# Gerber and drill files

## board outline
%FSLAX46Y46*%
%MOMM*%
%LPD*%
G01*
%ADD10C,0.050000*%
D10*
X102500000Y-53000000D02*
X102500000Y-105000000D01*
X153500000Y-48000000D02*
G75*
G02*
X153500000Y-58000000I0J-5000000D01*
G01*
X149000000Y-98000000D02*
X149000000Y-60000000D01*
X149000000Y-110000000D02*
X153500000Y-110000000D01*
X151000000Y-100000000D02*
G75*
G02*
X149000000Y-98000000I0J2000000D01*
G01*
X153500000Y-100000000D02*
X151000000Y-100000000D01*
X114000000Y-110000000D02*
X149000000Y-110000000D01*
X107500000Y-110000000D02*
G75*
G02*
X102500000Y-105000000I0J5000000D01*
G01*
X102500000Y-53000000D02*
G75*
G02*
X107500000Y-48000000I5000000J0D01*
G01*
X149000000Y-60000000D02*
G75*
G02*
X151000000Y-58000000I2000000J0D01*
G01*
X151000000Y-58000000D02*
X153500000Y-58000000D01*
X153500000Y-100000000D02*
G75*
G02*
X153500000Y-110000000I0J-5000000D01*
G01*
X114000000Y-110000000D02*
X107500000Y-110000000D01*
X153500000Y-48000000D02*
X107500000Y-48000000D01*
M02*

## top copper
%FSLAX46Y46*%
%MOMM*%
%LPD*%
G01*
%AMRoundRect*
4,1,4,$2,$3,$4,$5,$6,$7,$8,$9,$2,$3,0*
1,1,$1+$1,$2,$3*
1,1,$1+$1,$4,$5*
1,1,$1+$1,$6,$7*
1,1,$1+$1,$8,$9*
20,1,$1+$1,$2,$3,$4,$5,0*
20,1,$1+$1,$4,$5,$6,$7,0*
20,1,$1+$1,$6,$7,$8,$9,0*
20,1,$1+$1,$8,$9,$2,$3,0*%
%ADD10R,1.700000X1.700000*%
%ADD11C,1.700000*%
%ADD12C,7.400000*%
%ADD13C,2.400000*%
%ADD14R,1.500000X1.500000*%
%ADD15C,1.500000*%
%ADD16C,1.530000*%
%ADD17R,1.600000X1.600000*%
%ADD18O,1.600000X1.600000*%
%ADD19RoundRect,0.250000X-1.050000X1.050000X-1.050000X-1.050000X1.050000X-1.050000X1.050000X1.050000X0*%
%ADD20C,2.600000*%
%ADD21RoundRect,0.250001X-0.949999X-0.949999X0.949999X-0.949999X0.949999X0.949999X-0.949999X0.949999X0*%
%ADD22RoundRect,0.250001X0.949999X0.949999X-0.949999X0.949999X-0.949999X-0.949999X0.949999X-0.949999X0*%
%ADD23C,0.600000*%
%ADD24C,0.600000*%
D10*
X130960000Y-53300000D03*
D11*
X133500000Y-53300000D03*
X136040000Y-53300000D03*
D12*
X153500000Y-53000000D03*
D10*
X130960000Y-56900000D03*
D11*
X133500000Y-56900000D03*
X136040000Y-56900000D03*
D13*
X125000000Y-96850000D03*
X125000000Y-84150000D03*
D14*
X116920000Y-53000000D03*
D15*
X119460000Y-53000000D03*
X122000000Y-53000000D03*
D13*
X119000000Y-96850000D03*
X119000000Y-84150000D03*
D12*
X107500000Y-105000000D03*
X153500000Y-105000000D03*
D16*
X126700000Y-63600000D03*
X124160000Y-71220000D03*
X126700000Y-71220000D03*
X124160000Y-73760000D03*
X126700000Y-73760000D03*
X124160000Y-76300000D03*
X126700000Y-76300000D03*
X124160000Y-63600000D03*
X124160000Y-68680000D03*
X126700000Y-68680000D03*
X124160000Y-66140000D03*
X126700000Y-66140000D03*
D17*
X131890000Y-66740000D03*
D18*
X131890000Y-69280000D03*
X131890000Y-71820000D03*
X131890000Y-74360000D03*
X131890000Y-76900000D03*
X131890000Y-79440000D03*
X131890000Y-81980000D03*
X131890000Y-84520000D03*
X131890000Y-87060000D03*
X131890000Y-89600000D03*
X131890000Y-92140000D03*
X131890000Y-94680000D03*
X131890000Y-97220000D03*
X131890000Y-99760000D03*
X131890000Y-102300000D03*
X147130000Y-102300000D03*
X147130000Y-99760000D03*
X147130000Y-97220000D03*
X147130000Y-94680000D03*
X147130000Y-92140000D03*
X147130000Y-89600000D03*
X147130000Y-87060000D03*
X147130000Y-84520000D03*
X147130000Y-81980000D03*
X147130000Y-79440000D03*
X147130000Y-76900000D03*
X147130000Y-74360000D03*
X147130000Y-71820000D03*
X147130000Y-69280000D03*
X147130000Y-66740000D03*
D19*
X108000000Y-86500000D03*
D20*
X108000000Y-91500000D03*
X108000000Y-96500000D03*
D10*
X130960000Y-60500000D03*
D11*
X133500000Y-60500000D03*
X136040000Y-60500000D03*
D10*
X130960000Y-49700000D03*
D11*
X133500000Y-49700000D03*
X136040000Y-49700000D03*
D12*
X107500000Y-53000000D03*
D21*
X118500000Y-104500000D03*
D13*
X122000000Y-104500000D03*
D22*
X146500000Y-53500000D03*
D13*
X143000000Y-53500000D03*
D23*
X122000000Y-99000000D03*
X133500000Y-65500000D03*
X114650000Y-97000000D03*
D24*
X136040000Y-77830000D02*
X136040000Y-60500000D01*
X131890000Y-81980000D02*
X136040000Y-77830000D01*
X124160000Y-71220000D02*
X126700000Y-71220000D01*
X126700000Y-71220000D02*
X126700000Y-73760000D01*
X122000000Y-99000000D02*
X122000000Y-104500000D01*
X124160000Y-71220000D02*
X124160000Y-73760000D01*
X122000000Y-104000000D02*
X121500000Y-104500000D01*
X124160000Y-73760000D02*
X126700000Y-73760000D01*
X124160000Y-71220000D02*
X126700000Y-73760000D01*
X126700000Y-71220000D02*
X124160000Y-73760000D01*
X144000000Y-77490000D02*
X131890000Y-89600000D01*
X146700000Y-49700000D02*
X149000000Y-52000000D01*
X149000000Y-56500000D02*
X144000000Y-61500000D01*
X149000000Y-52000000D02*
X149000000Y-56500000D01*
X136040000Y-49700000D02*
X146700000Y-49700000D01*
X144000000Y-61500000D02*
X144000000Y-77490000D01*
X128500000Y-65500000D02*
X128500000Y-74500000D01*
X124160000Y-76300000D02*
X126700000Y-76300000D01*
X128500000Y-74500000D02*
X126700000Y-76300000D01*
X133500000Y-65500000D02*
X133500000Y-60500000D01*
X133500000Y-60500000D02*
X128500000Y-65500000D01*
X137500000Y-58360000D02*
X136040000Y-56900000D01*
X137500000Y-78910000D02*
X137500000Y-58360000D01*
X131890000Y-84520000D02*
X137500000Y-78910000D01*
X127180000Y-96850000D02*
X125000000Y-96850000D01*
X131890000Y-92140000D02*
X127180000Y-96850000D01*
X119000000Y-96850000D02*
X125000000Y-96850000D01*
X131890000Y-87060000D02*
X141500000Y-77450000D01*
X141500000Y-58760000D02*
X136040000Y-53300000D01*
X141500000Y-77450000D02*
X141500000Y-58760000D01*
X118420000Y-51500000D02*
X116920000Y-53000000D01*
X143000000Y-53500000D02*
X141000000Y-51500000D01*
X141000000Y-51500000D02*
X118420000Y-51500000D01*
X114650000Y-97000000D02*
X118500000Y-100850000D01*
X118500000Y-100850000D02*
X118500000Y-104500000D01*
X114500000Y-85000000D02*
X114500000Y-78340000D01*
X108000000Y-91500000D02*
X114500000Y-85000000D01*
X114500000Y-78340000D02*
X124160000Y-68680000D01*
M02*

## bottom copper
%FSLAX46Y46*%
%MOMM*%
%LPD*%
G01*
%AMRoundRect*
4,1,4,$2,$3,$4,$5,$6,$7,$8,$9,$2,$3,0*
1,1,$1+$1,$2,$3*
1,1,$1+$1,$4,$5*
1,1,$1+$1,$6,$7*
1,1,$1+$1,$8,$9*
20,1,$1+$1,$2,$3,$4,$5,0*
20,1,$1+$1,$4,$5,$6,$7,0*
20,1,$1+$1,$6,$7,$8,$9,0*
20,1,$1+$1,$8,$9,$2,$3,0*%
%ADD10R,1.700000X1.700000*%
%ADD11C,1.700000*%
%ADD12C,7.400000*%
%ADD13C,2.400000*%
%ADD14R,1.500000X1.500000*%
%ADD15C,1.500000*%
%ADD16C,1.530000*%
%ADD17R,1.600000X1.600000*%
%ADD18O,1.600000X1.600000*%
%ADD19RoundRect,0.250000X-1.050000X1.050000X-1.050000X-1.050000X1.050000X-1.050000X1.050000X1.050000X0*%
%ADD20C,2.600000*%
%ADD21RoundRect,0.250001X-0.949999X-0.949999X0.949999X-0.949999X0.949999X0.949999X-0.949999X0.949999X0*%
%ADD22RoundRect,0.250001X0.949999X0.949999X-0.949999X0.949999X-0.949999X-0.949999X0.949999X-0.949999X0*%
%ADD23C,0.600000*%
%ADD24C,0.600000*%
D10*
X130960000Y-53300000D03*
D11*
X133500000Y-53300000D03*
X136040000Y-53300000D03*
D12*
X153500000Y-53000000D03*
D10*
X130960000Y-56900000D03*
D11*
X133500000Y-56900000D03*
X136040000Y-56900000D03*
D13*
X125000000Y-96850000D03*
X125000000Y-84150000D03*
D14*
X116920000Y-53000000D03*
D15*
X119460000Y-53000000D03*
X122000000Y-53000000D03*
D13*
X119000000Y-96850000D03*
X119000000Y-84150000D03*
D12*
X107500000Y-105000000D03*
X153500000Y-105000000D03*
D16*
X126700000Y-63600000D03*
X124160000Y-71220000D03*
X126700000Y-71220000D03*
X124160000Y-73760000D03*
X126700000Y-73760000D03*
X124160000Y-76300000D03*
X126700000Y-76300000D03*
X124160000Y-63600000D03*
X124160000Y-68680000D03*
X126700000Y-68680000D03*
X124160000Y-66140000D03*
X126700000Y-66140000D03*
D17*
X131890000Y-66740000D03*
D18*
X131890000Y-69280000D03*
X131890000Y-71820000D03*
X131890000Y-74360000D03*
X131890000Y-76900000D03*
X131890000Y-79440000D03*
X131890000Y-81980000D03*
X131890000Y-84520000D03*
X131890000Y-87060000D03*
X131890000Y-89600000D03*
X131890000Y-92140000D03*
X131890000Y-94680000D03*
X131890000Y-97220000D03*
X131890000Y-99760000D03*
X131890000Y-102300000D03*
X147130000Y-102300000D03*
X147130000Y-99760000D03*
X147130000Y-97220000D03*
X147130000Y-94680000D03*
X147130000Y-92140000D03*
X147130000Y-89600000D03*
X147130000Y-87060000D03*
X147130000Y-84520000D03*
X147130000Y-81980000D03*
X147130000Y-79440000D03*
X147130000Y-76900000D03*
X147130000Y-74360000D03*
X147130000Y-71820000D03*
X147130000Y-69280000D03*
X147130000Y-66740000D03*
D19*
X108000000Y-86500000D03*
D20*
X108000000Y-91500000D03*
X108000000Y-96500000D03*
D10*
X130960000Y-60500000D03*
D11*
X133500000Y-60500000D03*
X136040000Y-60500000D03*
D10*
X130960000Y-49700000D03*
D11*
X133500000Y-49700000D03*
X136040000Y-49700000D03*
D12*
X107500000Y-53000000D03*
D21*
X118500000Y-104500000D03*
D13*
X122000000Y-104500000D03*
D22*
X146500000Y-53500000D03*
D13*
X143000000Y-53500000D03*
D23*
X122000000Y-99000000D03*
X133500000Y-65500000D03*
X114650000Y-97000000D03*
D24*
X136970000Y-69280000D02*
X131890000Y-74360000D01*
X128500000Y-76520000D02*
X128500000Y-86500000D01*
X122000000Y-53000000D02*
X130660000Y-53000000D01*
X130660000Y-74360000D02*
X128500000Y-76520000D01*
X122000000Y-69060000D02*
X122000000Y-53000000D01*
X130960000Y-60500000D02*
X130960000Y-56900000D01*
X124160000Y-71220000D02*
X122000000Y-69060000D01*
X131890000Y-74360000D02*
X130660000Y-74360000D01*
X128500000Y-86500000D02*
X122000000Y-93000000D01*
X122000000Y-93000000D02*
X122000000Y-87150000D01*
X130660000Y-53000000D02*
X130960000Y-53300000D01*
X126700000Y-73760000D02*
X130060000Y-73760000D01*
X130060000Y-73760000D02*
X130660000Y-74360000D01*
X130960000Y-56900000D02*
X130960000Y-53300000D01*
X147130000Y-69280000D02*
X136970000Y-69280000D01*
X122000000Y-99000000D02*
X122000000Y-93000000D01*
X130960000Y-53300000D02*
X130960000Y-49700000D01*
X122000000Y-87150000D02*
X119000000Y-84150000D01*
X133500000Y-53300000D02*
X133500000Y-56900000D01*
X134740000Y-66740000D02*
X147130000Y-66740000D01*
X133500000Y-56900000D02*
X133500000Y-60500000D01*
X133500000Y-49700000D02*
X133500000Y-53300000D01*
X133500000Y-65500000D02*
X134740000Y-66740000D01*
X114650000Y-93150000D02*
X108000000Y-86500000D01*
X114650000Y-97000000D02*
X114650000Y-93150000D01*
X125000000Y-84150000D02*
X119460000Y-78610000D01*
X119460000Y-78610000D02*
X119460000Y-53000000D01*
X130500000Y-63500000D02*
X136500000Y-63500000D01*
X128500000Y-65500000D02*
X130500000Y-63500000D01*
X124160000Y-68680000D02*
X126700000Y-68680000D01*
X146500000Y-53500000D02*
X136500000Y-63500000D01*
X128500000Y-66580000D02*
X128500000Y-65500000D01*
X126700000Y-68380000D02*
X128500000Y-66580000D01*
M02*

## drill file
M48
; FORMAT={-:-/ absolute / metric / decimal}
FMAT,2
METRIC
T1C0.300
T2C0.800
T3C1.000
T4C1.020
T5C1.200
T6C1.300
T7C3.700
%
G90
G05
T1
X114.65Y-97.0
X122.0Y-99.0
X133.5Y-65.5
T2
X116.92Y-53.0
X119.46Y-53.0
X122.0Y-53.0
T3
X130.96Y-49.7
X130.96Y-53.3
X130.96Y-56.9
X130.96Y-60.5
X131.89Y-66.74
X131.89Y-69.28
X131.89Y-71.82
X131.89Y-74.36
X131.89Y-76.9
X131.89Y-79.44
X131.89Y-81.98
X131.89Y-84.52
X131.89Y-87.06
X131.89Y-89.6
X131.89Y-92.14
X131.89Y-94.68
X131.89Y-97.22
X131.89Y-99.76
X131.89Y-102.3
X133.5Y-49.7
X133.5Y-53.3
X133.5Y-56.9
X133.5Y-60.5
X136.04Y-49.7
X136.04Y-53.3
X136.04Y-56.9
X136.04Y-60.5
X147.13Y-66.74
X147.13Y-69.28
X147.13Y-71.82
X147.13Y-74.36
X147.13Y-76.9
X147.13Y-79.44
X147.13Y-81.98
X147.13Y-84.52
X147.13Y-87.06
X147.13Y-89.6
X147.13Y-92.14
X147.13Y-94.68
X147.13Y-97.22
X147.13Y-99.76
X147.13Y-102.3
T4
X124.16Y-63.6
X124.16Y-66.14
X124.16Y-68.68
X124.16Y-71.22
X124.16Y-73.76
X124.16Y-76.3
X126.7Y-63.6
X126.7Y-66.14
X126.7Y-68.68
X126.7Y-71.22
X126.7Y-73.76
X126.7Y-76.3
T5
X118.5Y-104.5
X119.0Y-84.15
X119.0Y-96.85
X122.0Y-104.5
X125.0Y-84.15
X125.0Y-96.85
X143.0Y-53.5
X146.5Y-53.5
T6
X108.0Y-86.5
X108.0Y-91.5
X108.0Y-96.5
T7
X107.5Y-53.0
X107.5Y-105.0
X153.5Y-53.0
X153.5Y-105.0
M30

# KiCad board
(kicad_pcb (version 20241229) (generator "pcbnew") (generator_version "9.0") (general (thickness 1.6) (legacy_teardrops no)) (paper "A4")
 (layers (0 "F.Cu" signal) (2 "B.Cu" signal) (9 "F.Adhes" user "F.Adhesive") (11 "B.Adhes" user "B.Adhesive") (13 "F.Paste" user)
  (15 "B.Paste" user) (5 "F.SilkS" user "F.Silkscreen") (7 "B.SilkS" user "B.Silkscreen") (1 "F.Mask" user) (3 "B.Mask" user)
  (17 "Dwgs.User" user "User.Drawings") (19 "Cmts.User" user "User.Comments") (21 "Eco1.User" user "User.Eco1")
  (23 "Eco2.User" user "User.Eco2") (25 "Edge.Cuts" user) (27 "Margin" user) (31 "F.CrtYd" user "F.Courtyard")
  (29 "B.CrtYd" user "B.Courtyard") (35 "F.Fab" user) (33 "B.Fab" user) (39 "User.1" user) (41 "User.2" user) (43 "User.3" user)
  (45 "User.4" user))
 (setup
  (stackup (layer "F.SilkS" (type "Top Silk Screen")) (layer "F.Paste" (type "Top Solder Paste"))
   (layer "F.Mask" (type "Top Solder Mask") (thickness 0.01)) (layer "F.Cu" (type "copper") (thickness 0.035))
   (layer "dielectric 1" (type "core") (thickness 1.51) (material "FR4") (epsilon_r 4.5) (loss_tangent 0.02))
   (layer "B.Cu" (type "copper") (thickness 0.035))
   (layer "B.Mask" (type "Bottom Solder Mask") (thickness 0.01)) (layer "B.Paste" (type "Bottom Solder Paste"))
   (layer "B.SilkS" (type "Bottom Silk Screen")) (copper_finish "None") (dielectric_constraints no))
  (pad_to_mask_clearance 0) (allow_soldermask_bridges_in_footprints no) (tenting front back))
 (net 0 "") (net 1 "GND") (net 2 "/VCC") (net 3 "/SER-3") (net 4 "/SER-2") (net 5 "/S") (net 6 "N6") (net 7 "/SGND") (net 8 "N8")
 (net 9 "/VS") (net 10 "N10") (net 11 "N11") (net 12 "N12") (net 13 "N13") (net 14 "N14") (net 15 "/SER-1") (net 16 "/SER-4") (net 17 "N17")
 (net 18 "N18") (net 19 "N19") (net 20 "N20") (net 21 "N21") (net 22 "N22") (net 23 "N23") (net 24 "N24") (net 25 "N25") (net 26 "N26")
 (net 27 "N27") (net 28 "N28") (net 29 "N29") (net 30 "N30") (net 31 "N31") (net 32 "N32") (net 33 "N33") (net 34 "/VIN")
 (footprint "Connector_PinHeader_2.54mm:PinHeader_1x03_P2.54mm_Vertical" (layer "F.Cu") (at 130.96 53.3 90)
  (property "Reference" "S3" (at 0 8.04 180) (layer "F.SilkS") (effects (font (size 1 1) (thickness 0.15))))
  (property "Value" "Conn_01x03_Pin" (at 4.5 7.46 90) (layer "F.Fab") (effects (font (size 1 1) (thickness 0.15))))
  (pad "1" thru_hole rect (at 0 0 90) (size 1.7 1.7) (drill 1) (layers "*.Cu" "*.Mask") (remove_unused_layers no) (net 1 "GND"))
  (pad "2" thru_hole circle (at 0 2.54 90) (size 1.7 1.7) (drill 1) (layers "*.Cu" "*.Mask") (remove_unused_layers no) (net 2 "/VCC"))
  (pad "3" thru_hole circle (at 0 5.08 90) (size 1.7 1.7) (drill 1) (layers "*.Cu" "*.Mask") (remove_unused_layers no) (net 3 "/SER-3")))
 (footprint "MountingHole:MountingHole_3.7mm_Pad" (layer "F.Cu") (at 153.5 53)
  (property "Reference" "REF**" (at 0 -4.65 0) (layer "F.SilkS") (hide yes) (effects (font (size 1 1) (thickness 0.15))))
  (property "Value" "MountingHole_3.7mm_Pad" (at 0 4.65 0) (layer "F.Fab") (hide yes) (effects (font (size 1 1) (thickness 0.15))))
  (pad "1" thru_hole circle (at 0 0) (size 7.4 7.4) (drill 3.7) (layers "*.Cu" "*.Mask") (remove_unused_layers no) (zone_connect 2)))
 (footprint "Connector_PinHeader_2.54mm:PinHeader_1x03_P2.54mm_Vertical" (layer "F.Cu") (at 130.96 56.9 90)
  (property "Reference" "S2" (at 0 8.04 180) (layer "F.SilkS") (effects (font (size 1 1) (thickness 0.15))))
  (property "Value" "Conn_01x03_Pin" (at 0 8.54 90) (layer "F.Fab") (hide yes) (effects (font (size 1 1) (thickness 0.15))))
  (pad "1" thru_hole rect (at 0 0 90) (size 1.7 1.7) (drill 1) (layers "*.Cu" "*.Mask") (remove_unused_layers no) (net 1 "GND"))
  (pad "2" thru_hole circle (at 0 2.54 90) (size 1.7 1.7) (drill 1) (layers "*.Cu" "*.Mask") (remove_unused_layers no) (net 2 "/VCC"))
  (pad "3" thru_hole circle (at 0 5.08 90) (size 1.7 1.7) (drill 1) (layers "*.Cu" "*.Mask") (remove_unused_layers no) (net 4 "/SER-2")))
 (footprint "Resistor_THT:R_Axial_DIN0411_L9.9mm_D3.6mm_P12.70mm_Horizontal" (layer "F.Cu") (at 125 96.85 90)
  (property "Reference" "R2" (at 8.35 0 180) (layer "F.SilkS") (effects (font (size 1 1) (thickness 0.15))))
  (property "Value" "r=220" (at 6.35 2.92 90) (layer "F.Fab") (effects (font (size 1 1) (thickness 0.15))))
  (pad "1" thru_hole circle (at 0 0 90) (size 2.4 2.4) (drill 1.2) (layers "*.Cu" "*.Mask") (remove_unused_layers no) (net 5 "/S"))
  (pad "2" thru_hole circle (at 12.7 0 90) (size 2.4 2.4) (drill 1.2) (layers "*.Cu" "*.Mask") (remove_unused_layers no) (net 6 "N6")))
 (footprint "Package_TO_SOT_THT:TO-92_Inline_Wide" (layer "F.Cu") (at 116.92 53)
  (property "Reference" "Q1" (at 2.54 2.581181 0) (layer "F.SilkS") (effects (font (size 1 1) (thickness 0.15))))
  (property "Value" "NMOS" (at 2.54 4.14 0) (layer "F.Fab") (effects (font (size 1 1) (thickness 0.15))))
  (pad "1" thru_hole rect (at 0 0) (size 1.5 1.5) (drill 0.8) (layers "*.Cu" "*.Mask") (remove_unused_layers no) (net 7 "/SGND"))
  (pad "2" thru_hole circle (at 2.54 0) (size 1.5 1.5) (drill 0.8) (layers "*.Cu" "*.Mask") (remove_unused_layers no) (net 6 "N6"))
  (pad "3" thru_hole circle (at 5.08 0) (size 1.5 1.5) (drill 0.8) (layers "*.Cu" "*.Mask") (remove_unused_layers no) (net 1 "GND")))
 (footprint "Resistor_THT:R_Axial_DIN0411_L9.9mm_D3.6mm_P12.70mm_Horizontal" (layer "F.Cu") (at 119 96.85 90)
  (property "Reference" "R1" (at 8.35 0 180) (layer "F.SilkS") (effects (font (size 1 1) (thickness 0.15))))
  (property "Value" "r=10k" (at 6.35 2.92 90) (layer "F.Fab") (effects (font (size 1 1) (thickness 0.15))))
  (pad "1" thru_hole circle (at 0 0 90) (size 2.4 2.4) (drill 1.2) (layers "*.Cu" "*.Mask") (remove_unused_layers no) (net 5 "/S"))
  (pad "2" thru_hole circle (at 12.7 0 90) (size 2.4 2.4) (drill 1.2) (layers "*.Cu" "*.Mask") (remove_unused_layers no) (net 1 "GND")))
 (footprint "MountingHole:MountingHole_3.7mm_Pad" (layer "F.Cu") (at 107.5 105)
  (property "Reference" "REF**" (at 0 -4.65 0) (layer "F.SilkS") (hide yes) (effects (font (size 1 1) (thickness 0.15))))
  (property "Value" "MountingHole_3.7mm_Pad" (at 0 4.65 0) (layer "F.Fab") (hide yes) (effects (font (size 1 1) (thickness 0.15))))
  (pad "1" thru_hole circle (at 0 0) (size 7.4 7.4) (drill 3.7) (layers "*.Cu" "*.Mask") (remove_unused_layers no) (zone_connect 2)))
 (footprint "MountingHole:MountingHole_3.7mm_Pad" (layer "F.Cu") (at 153.5 105)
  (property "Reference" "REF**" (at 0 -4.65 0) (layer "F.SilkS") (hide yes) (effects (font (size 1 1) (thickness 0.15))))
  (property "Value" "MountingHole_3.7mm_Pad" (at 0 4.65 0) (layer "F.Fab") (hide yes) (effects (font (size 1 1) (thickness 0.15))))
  (pad "1" thru_hole circle (at 0 0) (size 7.4 7.4) (drill 3.7) (layers "*.Cu" "*.Mask") (remove_unused_layers no) (zone_connect 2)))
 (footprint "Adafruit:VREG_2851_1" (layer "F.Cu") (at 118 73.8)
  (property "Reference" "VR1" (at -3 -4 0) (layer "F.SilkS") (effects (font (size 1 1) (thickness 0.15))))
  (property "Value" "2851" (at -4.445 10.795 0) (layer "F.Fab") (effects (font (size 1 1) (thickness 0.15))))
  (pad "EN" thru_hole circle (at 8.7 -10.2) (size 1.53 1.53) (drill 1.02) (layers "*.Cu" "*.Mask") (remove_unused_layers no) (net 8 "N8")
   (solder_mask_margin 0.102))
  (pad "GND1" thru_hole circle (at 6.16 -2.58) (size 1.53 1.53) (drill 1.02) (layers "*.Cu" "*.Mask") (remove_unused_layers no)
   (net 1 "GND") (solder_mask_margin 0.102))
  (pad "GND1" thru_hole circle (at 8.7 -2.58) (size 1.53 1.53) (drill 1.02) (layers "*.Cu" "*.Mask") (remove_unused_layers no) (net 1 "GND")
   (solder_mask_margin 0.102))
  (pad "GND2" thru_hole circle (at 6.16 -0.04) (size 1.53 1.53) (drill 1.02) (layers "*.Cu" "*.Mask") (remove_unused_layers no)
   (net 1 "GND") (solder_mask_margin 0.102))
  (pad "GND2" thru_hole circle (at 8.7 -0.04) (size 1.53 1.53) (drill 1.02) (layers "*.Cu" "*.Mask") (remove_unused_layers no) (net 1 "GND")
   (solder_mask_margin 0.102))
  (pad "OUT" thru_hole circle (at 6.16 2.5) (size 1.53 1.53) (drill 1.02) (layers "*.Cu" "*.Mask") (remove_unused_layers no) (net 2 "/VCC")
   (solder_mask_margin 0.102))
  (pad "OUT" thru_hole circle (at 8.7 2.5) (size 1.53 1.53) (drill 1.02) (layers "*.Cu" "*.Mask") (remove_unused_layers no) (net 2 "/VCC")
   (solder_mask_margin 0.102))
  (pad "PG" thru_hole circle (at 6.16 -10.2) (size 1.53 1.53) (drill 1.02) (layers "*.Cu" "*.Mask") (remove_unused_layers no)
   (solder_mask_margin 0.102))
  (pad "VIN" thru_hole circle (at 6.16 -5.12) (size 1.53 1.53) (drill 1.02) (layers "*.Cu" "*.Mask") (remove_unused_layers no) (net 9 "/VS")
   (solder_mask_margin 0.102))
  (pad "VIN" thru_hole circle (at 8.7 -5.12) (size 1.53 1.53) (drill 1.02) (layers "*.Cu" "*.Mask") (remove_unused_layers no) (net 9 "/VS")
   (solder_mask_margin 0.102))
  (pad "VRP" thru_hole circle (at 6.16 -7.66) (size 1.53 1.53) (drill 1.02) (layers "*.Cu" "*.Mask") (remove_unused_layers no)
   (solder_mask_margin 0.102))
  (pad "VRP" thru_hole circle (at 8.7 -7.66) (size 1.53 1.53) (drill 1.02) (layers "*.Cu" "*.Mask") (remove_unused_layers no)
   (solder_mask_margin 0.102)))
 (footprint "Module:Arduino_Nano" (layer "F.Cu") (at 131.89 66.74)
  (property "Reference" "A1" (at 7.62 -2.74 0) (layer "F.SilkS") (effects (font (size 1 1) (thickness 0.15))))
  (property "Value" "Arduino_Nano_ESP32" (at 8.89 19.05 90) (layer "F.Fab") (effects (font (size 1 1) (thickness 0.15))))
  (pad "1" thru_hole rect (at 0 0) (size 1.6 1.6) (drill 1) (layers "*.Cu" "*.Mask") (remove_unused_layers no) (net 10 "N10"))
  (pad "2" thru_hole oval (at 0 2.54) (size 1.6 1.6) (drill 1) (layers "*.Cu" "*.Mask") (remove_unused_layers no) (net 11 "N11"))
  (pad "3" thru_hole oval (at 0 5.08) (size 1.6 1.6) (drill 1) (layers "*.Cu" "*.Mask") (remove_unused_layers no) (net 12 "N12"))
  (pad "4" thru_hole oval (at 0 7.62) (size 1.6 1.6) (drill 1) (layers "*.Cu" "*.Mask") (remove_unused_layers no) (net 1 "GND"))
  (pad "5" thru_hole oval (at 0 10.16) (size 1.6 1.6) (drill 1) (layers "*.Cu" "*.Mask") (remove_unused_layers no) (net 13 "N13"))
  (pad "6" thru_hole oval (at 0 12.7) (size 1.6 1.6) (drill 1) (layers "*.Cu" "*.Mask") (remove_unused_layers no) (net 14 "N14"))
  (pad "7" thru_hole oval (at 0 15.24) (size 1.6 1.6) (drill 1) (layers "*.Cu" "*.Mask") (remove_unused_layers no) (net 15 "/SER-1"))
  (pad "8" thru_hole oval (at 0 17.78) (size 1.6 1.6) (drill 1) (layers "*.Cu" "*.Mask") (remove_unused_layers no) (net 4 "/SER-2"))
  (pad "9" thru_hole oval (at 0 20.32) (size 1.6 1.6) (drill 1) (layers "*.Cu" "*.Mask") (remove_unused_layers no) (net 3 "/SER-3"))
  (pad "10" thru_hole oval (at 0 22.86) (size 1.6 1.6) (drill 1) (layers "*.Cu" "*.Mask") (remove_unused_layers no) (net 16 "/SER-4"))
  (pad "11" thru_hole oval (at 0 25.4) (size 1.6 1.6) (drill 1) (layers "*.Cu" "*.Mask") (remove_unused_layers no) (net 5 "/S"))
  (pad "12" thru_hole oval (at 0 27.94) (size 1.6 1.6) (drill 1) (layers "*.Cu" "*.Mask") (remove_unused_layers no) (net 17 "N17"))
  (pad "13" thru_hole oval (at 0 30.48) (size 1.6 1.6) (drill 1) (layers "*.Cu" "*.Mask") (remove_unused_layers no) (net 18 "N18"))
  (pad "14" thru_hole oval (at 0 33.02) (size 1.6 1.6) (drill 1) (layers "*.Cu" "*.Mask") (remove_unused_layers no) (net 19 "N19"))
  (pad "15" thru_hole oval (at 0 35.56) (size 1.6 1.6) (drill 1) (layers "*.Cu" "*.Mask") (remove_unused_layers no) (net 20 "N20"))
  (pad "16" thru_hole oval (at 15.24 35.56) (size 1.6 1.6) (drill 1) (layers "*.Cu" "*.Mask") (remove_unused_layers no) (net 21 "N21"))
  (pad "17" thru_hole oval (at 15.24 33.02) (size 1.6 1.6) (drill 1) (layers "*.Cu" "*.Mask") (remove_unused_layers no) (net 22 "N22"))
  (pad "18" thru_hole oval (at 15.24 30.48) (size 1.6 1.6) (drill 1) (layers "*.Cu" "*.Mask") (remove_unused_layers no) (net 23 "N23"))
  (pad "19" thru_hole oval (at 15.24 27.94) (size 1.6 1.6) (drill 1) (layers "*.Cu" "*.Mask") (remove_unused_layers no) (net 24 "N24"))
  (pad "20" thru_hole oval (at 15.24 25.4) (size 1.6 1.6) (drill 1) (layers "*.Cu" "*.Mask") (remove_unused_layers no) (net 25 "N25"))
  (pad "21" thru_hole oval (at 15.24 22.86) (size 1.6 1.6) (drill 1) (layers "*.Cu" "*.Mask") (remove_unused_layers no) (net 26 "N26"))
  (pad "22" thru_hole oval (at 15.24 20.32) (size 1.6 1.6) (drill 1) (layers "*.Cu" "*.Mask") (remove_unused_layers no) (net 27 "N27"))
  (pad "23" thru_hole oval (at 15.24 17.78) (size 1.6 1.6) (drill 1) (layers "*.Cu" "*.Mask") (remove_unused_layers no) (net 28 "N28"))
  (pad "24" thru_hole oval (at 15.24 15.24) (size 1.6 1.6) (drill 1) (layers "*.Cu" "*.Mask") (remove_unused_layers no) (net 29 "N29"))
  (pad "25" thru_hole oval (at 15.24 12.7) (size 1.6 1.6) (drill 1) (layers "*.Cu" "*.Mask") (remove_unused_layers no) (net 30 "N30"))
  (pad "26" thru_hole oval (at 15.24 10.16) (size 1.6 1.6) (drill 1) (layers "*.Cu" "*.Mask") (remove_unused_layers no) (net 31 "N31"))
  (pad "27" thru_hole oval (at 15.24 7.62) (size 1.6 1.6) (drill 1) (layers "*.Cu" "*.Mask") (remove_unused_layers no) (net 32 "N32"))
  (pad "28" thru_hole oval (at 15.24 5.08) (size 1.6 1.6) (drill 1) (layers "*.Cu" "*.Mask") (remove_unused_layers no) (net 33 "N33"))
  (pad "29" thru_hole oval (at 15.24 2.54) (size 1.6 1.6) (drill 1) (layers "*.Cu" "*.Mask") (remove_unused_layers no) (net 1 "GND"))
  (pad "30" thru_hole oval (at 15.24 0) (size 1.6 1.6) (drill 1) (layers "*.Cu" "*.Mask") (remove_unused_layers no) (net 2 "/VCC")))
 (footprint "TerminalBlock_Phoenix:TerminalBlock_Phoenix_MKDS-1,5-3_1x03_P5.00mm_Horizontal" (layer "F.Cu") (at 108 86.5 -90)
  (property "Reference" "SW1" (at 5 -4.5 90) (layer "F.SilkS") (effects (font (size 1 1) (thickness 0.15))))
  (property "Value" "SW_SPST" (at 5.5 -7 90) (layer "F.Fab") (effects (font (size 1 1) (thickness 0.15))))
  (pad "1" thru_hole roundrect (at 0 0 270) (size 2.6 2.6) (drill 1.3) (layers "*.Cu" "*.Mask") (remove_unused_layers no)
   (roundrect_rratio 0.096154) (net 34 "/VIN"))
  (pad "2" thru_hole circle (at 5 0 270) (size 2.6 2.6) (drill 1.3) (layers "*.Cu" "*.Mask") (remove_unused_layers no) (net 9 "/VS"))
  (pad "3" thru_hole circle (at 10 0 270) (size 2.6 2.6) (drill 1.3) (layers "*.Cu" "*.Mask") (remove_unused_layers no)))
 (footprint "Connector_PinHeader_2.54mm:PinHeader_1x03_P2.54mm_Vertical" (layer "F.Cu") (at 130.96 60.5 90)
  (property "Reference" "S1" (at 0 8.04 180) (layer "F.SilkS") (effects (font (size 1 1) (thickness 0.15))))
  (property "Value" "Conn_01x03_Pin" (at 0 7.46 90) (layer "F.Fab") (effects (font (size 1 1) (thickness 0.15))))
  (pad "1" thru_hole rect (at 0 0 90) (size 1.7 1.7) (drill 1) (layers "*.Cu" "*.Mask") (remove_unused_layers no) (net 1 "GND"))
  (pad "2" thru_hole circle (at 0 2.54 90) (size 1.7 1.7) (drill 1) (layers "*.Cu" "*.Mask") (remove_unused_layers no) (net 2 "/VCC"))
  (pad "3" thru_hole circle (at 0 5.08 90) (size 1.7 1.7) (drill 1) (layers "*.Cu" "*.Mask") (remove_unused_layers no) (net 15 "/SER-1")))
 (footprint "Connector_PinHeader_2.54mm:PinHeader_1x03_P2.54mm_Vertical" (layer "F.Cu") (at 130.96 49.7 90)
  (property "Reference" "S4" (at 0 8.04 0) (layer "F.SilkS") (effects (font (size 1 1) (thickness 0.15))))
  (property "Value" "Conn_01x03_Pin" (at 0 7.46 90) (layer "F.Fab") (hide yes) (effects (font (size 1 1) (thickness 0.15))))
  (pad "1" thru_hole rect (at 0 0 90) (size 1.7 1.7) (drill 1) (layers "*.Cu" "*.Mask") (remove_unused_layers no) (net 1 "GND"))
  (pad "2" thru_hole circle (at 0 2.54 90) (size 1.7 1.7) (drill 1) (layers "*.Cu" "*.Mask") (remove_unused_layers no) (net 2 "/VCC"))
  (pad "3" thru_hole circle (at 0 5.08 90) (size 1.7 1.7) (drill 1) (layers "*.Cu" "*.Mask") (remove_unused_layers no) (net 16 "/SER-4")))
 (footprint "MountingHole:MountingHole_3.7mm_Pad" (layer "F.Cu") (at 107.5 53)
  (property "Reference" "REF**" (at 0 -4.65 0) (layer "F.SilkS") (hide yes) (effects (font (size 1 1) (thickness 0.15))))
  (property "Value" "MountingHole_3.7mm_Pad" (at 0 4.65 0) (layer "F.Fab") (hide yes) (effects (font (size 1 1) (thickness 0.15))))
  (pad "1" thru_hole circle (at 0 0) (size 7.4 7.4) (drill 3.7) (layers "*.Cu" "*.Mask") (remove_unused_layers no) (zone_connect 2)))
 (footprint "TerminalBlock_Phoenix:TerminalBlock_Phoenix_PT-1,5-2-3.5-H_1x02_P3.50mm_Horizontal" (layer "F.Cu") (at 118.5 104.5)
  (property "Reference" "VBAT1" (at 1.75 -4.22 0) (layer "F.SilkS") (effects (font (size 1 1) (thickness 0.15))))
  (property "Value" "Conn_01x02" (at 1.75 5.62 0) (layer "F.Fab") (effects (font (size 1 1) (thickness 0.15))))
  (pad "1" thru_hole roundrect (at 0 0) (size 2.4 2.4) (drill 1.2) (layers "*.Cu" "*.Mask") (remove_unused_layers no)
   (roundrect_rratio 0.104167) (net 34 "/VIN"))
  (pad "2" thru_hole circle (at 3.5 0) (size 2.4 2.4) (drill 1.2) (layers "*.Cu" "*.Mask") (remove_unused_layers no) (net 1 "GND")))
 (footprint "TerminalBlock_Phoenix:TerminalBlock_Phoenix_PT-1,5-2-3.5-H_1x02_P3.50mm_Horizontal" (layer "F.Cu") (at 146.5 53.5 180)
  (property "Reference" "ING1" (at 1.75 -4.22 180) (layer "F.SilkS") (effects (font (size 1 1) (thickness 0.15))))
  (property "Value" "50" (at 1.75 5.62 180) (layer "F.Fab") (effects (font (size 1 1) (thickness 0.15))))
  (pad "1" thru_hole roundrect (at 0 0 180) (size 2.4 2.4) (drill 1.2) (layers "*.Cu" "*.Mask") (remove_unused_layers no)
   (roundrect_rratio 0.104167) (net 9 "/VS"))
  (pad "2" thru_hole circle (at 3.5 0 180) (size 2.4 2.4) (drill 1.2) (layers "*.Cu" "*.Mask") (remove_unused_layers no) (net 7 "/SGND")))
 (gr_line (start 102.5 53) (end 102.5 105) (stroke (width 0.05) (type solid)) (layer "Edge.Cuts"))
 (gr_arc (start 153.5 48) (mid 158.5 53) (end 153.5 58) (stroke (width 0.05) (type default)) (layer "Edge.Cuts"))
 (gr_line (start 149 98) (end 149 60) (stroke (width 0.05) (type default)) (layer "Edge.Cuts"))
 (gr_line (start 149 110) (end 153.5 110) (stroke (width 0.05) (type default)) (layer "Edge.Cuts"))
 (gr_arc (start 151 100) (mid 149.585786 99.414214) (end 149 98) (stroke (width 0.05) (type default)) (layer "Edge.Cuts"))
 (gr_line (start 153.5 100) (end 151 100) (stroke (width 0.05) (type default)) (layer "Edge.Cuts"))
 (gr_line (start 114 110) (end 149 110) (stroke (width 0.05) (type default)) (layer "Edge.Cuts"))
 (gr_arc (start 107.5 110) (mid 103.964466 108.535534) (end 102.5 105) (stroke (width 0.05) (type default)) (layer "Edge.Cuts"))
 (gr_arc (start 102.5 53) (mid 103.964466 49.464466) (end 107.5 48) (stroke (width 0.05) (type default)) (layer "Edge.Cuts"))
 (gr_arc (start 149 60) (mid 149.585786 58.585786) (end 151 58) (stroke (width 0.05) (type default)) (layer "Edge.Cuts"))
 (gr_line (start 151 58) (end 153.5 58) (stroke (width 0.05) (type default)) (layer "Edge.Cuts"))
 (gr_arc (start 153.5 100) (mid 158.5 105) (end 153.5 110) (stroke (width 0.05) (type default)) (layer "Edge.Cuts"))
 (gr_line (start 114 110) (end 107.5 110) (stroke (width 0.05) (type default)) (layer "Edge.Cuts"))
 (gr_line (start 153.5 48) (end 107.5 48) (stroke (width 0.05) (type default)) (layer "Edge.Cuts"))
 (segment (start 136.04 77.83) (end 136.04 60.5) (width 0.6) (layer "F.Cu") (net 15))
 (segment (start 131.89 81.98) (end 136.04 77.83) (width 0.6) (layer "F.Cu") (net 15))
 (segment (start 124.16 71.22) (end 126.7 71.22) (width 0.6) (layer "F.Cu") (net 1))
 (segment (start 126.7 71.22) (end 126.7 73.76) (width 0.6) (layer "F.Cu") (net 1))
 (segment (start 122 99) (end 122 104.5) (width 0.6) (layer "F.Cu") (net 1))
 (segment (start 124.16 71.22) (end 124.16 73.76) (width 0.6) (layer "F.Cu") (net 1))
 (segment (start 122 104) (end 121.5 104.5) (width 0.6) (layer "F.Cu") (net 1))
 (segment (start 124.16 73.76) (end 126.7 73.76) (width 0.6) (layer "F.Cu") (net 1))
 (segment (start 124.16 71.22) (end 126.7 73.76) (width 0.6) (layer "F.Cu") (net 1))
 (segment (start 126.7 71.22) (end 124.16 73.76) (width 0.6) (layer "F.Cu") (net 1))
 (via (at 122 99) (size 0.6) (drill 0.3) (layers "F.Cu" "B.Cu") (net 1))
 (segment (start 136.97 69.28) (end 131.89 74.36) (width 0.6) (layer "B.Cu") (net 1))
 (segment (start 128.5 76.52) (end 128.5 86.5) (width 0.6) (layer "B.Cu") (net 1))
 (segment (start 122 53) (end 130.66 53) (width 0.6) (layer "B.Cu") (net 1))
 (segment (start 130.66 74.36) (end 128.5 76.52) (width 0.6) (layer "B.Cu") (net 1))
 (segment (start 122 69.06) (end 122 53) (width 0.6) (layer "B.Cu") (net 1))
 (segment (start 130.96 60.5) (end 130.96 56.9) (width 0.6) (layer "B.Cu") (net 1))
 (segment (start 124.16 71.22) (end 122 69.06) (width 0.6) (layer "B.Cu") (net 1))
 (segment (start 131.89 74.36) (end 130.66 74.36) (width 0.6) (layer "B.Cu") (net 1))
 (segment (start 128.5 86.5) (end 122 93) (width 0.6) (layer "B.Cu") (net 1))
 (segment (start 122 93) (end 122 87.15) (width 0.6) (layer "B.Cu") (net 1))
 (segment (start 130.66 53) (end 130.96 53.3) (width 0.6) (layer "B.Cu") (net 1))
 (segment (start 126.7 73.76) (end 130.06 73.76) (width 0.6) (layer "B.Cu") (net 1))
 (segment (start 130.06 73.76) (end 130.66 74.36) (width 0.6) (layer "B.Cu") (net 1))
 (segment (start 130.96 56.9) (end 130.96 53.3) (width 0.6) (layer "B.Cu") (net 1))
 (segment (start 147.13 69.28) (end 136.97 69.28) (width 0.6) (layer "B.Cu") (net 1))
 (segment (start 122 99) (end 122 93) (width 0.6) (layer "B.Cu") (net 1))
 (segment (start 130.96 53.3) (end 130.96 49.7) (width 0.6) (layer "B.Cu") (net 1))
 (segment (start 122 87.15) (end 119 84.15) (width 0.6) (layer "B.Cu") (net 1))
 (segment (start 144 77.49) (end 131.89 89.6) (width 0.6) (layer "F.Cu") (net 16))
 (segment (start 146.7 49.7) (end 149 52) (width 0.6) (layer "F.Cu") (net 16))
 (segment (start 149 56.5) (end 144 61.5) (width 0.6) (layer "F.Cu") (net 16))
 (segment (start 149 52) (end 149 56.5) (width 0.6) (layer "F.Cu") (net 16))
 (segment (start 136.04 49.7) (end 146.7 49.7) (width 0.6) (layer "F.Cu") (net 16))
 (segment (start 144 61.5) (end 144 77.49) (width 0.6) (layer "F.Cu") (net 16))
 (segment (start 128.5 65.5) (end 128.5 74.5) (width 0.6) (layer "F.Cu") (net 2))
 (segment (start 124.16 76.3) (end 126.7 76.3) (width 0.6) (layer "F.Cu") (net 2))
 (segment (start 128.5 74.5) (end 126.7 76.3) (width 0.6) (layer "F.Cu") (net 2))
 (segment (start 133.5 65.5) (end 133.5 60.5) (width 0.6) (layer "F.Cu") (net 2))
 (segment (start 133.5 60.5) (end 128.5 65.5) (width 0.6) (layer "F.Cu") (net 2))
 (via (at 133.5 65.5) (size 0.6) (drill 0.3) (layers "F.Cu" "B.Cu") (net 2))
 (segment (start 133.5 53.3) (end 133.5 56.9) (width 0.6) (layer "B.Cu") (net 2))
 (segment (start 134.74 66.74) (end 147.13 66.74) (width 0.6) (layer "B.Cu") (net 2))
 (segment (start 133.5 56.9) (end 133.5 60.5) (width 0.6) (layer "B.Cu") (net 2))
 (segment (start 133.5 49.7) (end 133.5 53.3) (width 0.6) (layer "B.Cu") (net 2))
 (segment (start 133.5 65.5) (end 134.74 66.74) (width 0.6) (layer "B.Cu") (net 2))
 (segment (start 137.5 58.36) (end 136.04 56.9) (width 0.6) (layer "F.Cu") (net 4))
 (segment (start 137.5 78.91) (end 137.5 58.36) (width 0.6) (layer "F.Cu") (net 4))
 (segment (start 131.89 84.52) (end 137.5 78.91) (width 0.6) (layer "F.Cu") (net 4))
 (segment (start 127.18 96.85) (end 125 96.85) (width 0.6) (layer "F.Cu") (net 5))
 (segment (start 131.89 92.14) (end 127.18 96.85) (width 0.6) (layer "F.Cu") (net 5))
 (segment (start 119 96.85) (end 125 96.85) (width 0.6) (layer "F.Cu") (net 5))
 (segment (start 131.89 87.06) (end 141.5 77.45) (width 0.6) (layer "F.Cu") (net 3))
 (segment (start 141.5 58.76) (end 136.04 53.3) (width 0.6) (layer "F.Cu") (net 3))
 (segment (start 141.5 77.45) (end 141.5 58.76) (width 0.6) (layer "F.Cu") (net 3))
 (segment (start 118.42 51.5) (end 116.92 53) (width 0.6) (layer "F.Cu") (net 7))
 (segment (start 143 53.5) (end 141 51.5) (width 0.6) (layer "F.Cu") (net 7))
 (segment (start 141 51.5) (end 118.42 51.5) (width 0.6) (layer "F.Cu") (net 7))
 (segment (start 114.65 97) (end 118.5 100.85) (width 0.6) (layer "F.Cu") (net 34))
 (segment (start 118.5 100.85) (end 118.5 104.5) (width 0.6) (layer "F.Cu") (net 34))
 (via (at 114.65 97) (size 0.6) (drill 0.3) (layers "F.Cu" "B.Cu") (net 34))
 (segment (start 114.65 93.15) (end 108 86.5) (width 0.6) (layer "B.Cu") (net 34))
 (segment (start 114.65 97) (end 114.65 93.15) (width 0.6) (layer "B.Cu") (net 34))
 (segment (start 125 84.15) (end 119.46 78.61) (width 0.6) (layer "B.Cu") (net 6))
 (segment (start 119.46 78.61) (end 119.46 53) (width 0.6) (layer "B.Cu") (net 6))
 (segment (start 114.5 85) (end 114.5 78.34) (width 0.6) (layer "F.Cu") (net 9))
 (segment (start 108 91.5) (end 114.5 85) (width 0.6) (layer "F.Cu") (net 9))
 (segment (start 114.5 78.34) (end 124.16 68.68) (width 0.6) (layer "F.Cu") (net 9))
 (segment (start 130.5 63.5) (end 136.5 63.5) (width 0.6) (layer "B.Cu") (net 9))
 (segment (start 128.5 65.5) (end 130.5 63.5) (width 0.6) (layer "B.Cu") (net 9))
 (segment (start 124.16 68.68) (end 126.7 68.68) (width 0.6) (layer "B.Cu") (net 9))
 (segment (start 146.5 53.5) (end 136.5 63.5) (width 0.6) (layer "B.Cu") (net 9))
 (segment (start 128.5 66.58) (end 128.5 65.5) (width 0.6) (layer "B.Cu") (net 9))
 (segment (start 126.7 68.38) (end 128.5 66.58) (width 0.6) (layer "B.Cu") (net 9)))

